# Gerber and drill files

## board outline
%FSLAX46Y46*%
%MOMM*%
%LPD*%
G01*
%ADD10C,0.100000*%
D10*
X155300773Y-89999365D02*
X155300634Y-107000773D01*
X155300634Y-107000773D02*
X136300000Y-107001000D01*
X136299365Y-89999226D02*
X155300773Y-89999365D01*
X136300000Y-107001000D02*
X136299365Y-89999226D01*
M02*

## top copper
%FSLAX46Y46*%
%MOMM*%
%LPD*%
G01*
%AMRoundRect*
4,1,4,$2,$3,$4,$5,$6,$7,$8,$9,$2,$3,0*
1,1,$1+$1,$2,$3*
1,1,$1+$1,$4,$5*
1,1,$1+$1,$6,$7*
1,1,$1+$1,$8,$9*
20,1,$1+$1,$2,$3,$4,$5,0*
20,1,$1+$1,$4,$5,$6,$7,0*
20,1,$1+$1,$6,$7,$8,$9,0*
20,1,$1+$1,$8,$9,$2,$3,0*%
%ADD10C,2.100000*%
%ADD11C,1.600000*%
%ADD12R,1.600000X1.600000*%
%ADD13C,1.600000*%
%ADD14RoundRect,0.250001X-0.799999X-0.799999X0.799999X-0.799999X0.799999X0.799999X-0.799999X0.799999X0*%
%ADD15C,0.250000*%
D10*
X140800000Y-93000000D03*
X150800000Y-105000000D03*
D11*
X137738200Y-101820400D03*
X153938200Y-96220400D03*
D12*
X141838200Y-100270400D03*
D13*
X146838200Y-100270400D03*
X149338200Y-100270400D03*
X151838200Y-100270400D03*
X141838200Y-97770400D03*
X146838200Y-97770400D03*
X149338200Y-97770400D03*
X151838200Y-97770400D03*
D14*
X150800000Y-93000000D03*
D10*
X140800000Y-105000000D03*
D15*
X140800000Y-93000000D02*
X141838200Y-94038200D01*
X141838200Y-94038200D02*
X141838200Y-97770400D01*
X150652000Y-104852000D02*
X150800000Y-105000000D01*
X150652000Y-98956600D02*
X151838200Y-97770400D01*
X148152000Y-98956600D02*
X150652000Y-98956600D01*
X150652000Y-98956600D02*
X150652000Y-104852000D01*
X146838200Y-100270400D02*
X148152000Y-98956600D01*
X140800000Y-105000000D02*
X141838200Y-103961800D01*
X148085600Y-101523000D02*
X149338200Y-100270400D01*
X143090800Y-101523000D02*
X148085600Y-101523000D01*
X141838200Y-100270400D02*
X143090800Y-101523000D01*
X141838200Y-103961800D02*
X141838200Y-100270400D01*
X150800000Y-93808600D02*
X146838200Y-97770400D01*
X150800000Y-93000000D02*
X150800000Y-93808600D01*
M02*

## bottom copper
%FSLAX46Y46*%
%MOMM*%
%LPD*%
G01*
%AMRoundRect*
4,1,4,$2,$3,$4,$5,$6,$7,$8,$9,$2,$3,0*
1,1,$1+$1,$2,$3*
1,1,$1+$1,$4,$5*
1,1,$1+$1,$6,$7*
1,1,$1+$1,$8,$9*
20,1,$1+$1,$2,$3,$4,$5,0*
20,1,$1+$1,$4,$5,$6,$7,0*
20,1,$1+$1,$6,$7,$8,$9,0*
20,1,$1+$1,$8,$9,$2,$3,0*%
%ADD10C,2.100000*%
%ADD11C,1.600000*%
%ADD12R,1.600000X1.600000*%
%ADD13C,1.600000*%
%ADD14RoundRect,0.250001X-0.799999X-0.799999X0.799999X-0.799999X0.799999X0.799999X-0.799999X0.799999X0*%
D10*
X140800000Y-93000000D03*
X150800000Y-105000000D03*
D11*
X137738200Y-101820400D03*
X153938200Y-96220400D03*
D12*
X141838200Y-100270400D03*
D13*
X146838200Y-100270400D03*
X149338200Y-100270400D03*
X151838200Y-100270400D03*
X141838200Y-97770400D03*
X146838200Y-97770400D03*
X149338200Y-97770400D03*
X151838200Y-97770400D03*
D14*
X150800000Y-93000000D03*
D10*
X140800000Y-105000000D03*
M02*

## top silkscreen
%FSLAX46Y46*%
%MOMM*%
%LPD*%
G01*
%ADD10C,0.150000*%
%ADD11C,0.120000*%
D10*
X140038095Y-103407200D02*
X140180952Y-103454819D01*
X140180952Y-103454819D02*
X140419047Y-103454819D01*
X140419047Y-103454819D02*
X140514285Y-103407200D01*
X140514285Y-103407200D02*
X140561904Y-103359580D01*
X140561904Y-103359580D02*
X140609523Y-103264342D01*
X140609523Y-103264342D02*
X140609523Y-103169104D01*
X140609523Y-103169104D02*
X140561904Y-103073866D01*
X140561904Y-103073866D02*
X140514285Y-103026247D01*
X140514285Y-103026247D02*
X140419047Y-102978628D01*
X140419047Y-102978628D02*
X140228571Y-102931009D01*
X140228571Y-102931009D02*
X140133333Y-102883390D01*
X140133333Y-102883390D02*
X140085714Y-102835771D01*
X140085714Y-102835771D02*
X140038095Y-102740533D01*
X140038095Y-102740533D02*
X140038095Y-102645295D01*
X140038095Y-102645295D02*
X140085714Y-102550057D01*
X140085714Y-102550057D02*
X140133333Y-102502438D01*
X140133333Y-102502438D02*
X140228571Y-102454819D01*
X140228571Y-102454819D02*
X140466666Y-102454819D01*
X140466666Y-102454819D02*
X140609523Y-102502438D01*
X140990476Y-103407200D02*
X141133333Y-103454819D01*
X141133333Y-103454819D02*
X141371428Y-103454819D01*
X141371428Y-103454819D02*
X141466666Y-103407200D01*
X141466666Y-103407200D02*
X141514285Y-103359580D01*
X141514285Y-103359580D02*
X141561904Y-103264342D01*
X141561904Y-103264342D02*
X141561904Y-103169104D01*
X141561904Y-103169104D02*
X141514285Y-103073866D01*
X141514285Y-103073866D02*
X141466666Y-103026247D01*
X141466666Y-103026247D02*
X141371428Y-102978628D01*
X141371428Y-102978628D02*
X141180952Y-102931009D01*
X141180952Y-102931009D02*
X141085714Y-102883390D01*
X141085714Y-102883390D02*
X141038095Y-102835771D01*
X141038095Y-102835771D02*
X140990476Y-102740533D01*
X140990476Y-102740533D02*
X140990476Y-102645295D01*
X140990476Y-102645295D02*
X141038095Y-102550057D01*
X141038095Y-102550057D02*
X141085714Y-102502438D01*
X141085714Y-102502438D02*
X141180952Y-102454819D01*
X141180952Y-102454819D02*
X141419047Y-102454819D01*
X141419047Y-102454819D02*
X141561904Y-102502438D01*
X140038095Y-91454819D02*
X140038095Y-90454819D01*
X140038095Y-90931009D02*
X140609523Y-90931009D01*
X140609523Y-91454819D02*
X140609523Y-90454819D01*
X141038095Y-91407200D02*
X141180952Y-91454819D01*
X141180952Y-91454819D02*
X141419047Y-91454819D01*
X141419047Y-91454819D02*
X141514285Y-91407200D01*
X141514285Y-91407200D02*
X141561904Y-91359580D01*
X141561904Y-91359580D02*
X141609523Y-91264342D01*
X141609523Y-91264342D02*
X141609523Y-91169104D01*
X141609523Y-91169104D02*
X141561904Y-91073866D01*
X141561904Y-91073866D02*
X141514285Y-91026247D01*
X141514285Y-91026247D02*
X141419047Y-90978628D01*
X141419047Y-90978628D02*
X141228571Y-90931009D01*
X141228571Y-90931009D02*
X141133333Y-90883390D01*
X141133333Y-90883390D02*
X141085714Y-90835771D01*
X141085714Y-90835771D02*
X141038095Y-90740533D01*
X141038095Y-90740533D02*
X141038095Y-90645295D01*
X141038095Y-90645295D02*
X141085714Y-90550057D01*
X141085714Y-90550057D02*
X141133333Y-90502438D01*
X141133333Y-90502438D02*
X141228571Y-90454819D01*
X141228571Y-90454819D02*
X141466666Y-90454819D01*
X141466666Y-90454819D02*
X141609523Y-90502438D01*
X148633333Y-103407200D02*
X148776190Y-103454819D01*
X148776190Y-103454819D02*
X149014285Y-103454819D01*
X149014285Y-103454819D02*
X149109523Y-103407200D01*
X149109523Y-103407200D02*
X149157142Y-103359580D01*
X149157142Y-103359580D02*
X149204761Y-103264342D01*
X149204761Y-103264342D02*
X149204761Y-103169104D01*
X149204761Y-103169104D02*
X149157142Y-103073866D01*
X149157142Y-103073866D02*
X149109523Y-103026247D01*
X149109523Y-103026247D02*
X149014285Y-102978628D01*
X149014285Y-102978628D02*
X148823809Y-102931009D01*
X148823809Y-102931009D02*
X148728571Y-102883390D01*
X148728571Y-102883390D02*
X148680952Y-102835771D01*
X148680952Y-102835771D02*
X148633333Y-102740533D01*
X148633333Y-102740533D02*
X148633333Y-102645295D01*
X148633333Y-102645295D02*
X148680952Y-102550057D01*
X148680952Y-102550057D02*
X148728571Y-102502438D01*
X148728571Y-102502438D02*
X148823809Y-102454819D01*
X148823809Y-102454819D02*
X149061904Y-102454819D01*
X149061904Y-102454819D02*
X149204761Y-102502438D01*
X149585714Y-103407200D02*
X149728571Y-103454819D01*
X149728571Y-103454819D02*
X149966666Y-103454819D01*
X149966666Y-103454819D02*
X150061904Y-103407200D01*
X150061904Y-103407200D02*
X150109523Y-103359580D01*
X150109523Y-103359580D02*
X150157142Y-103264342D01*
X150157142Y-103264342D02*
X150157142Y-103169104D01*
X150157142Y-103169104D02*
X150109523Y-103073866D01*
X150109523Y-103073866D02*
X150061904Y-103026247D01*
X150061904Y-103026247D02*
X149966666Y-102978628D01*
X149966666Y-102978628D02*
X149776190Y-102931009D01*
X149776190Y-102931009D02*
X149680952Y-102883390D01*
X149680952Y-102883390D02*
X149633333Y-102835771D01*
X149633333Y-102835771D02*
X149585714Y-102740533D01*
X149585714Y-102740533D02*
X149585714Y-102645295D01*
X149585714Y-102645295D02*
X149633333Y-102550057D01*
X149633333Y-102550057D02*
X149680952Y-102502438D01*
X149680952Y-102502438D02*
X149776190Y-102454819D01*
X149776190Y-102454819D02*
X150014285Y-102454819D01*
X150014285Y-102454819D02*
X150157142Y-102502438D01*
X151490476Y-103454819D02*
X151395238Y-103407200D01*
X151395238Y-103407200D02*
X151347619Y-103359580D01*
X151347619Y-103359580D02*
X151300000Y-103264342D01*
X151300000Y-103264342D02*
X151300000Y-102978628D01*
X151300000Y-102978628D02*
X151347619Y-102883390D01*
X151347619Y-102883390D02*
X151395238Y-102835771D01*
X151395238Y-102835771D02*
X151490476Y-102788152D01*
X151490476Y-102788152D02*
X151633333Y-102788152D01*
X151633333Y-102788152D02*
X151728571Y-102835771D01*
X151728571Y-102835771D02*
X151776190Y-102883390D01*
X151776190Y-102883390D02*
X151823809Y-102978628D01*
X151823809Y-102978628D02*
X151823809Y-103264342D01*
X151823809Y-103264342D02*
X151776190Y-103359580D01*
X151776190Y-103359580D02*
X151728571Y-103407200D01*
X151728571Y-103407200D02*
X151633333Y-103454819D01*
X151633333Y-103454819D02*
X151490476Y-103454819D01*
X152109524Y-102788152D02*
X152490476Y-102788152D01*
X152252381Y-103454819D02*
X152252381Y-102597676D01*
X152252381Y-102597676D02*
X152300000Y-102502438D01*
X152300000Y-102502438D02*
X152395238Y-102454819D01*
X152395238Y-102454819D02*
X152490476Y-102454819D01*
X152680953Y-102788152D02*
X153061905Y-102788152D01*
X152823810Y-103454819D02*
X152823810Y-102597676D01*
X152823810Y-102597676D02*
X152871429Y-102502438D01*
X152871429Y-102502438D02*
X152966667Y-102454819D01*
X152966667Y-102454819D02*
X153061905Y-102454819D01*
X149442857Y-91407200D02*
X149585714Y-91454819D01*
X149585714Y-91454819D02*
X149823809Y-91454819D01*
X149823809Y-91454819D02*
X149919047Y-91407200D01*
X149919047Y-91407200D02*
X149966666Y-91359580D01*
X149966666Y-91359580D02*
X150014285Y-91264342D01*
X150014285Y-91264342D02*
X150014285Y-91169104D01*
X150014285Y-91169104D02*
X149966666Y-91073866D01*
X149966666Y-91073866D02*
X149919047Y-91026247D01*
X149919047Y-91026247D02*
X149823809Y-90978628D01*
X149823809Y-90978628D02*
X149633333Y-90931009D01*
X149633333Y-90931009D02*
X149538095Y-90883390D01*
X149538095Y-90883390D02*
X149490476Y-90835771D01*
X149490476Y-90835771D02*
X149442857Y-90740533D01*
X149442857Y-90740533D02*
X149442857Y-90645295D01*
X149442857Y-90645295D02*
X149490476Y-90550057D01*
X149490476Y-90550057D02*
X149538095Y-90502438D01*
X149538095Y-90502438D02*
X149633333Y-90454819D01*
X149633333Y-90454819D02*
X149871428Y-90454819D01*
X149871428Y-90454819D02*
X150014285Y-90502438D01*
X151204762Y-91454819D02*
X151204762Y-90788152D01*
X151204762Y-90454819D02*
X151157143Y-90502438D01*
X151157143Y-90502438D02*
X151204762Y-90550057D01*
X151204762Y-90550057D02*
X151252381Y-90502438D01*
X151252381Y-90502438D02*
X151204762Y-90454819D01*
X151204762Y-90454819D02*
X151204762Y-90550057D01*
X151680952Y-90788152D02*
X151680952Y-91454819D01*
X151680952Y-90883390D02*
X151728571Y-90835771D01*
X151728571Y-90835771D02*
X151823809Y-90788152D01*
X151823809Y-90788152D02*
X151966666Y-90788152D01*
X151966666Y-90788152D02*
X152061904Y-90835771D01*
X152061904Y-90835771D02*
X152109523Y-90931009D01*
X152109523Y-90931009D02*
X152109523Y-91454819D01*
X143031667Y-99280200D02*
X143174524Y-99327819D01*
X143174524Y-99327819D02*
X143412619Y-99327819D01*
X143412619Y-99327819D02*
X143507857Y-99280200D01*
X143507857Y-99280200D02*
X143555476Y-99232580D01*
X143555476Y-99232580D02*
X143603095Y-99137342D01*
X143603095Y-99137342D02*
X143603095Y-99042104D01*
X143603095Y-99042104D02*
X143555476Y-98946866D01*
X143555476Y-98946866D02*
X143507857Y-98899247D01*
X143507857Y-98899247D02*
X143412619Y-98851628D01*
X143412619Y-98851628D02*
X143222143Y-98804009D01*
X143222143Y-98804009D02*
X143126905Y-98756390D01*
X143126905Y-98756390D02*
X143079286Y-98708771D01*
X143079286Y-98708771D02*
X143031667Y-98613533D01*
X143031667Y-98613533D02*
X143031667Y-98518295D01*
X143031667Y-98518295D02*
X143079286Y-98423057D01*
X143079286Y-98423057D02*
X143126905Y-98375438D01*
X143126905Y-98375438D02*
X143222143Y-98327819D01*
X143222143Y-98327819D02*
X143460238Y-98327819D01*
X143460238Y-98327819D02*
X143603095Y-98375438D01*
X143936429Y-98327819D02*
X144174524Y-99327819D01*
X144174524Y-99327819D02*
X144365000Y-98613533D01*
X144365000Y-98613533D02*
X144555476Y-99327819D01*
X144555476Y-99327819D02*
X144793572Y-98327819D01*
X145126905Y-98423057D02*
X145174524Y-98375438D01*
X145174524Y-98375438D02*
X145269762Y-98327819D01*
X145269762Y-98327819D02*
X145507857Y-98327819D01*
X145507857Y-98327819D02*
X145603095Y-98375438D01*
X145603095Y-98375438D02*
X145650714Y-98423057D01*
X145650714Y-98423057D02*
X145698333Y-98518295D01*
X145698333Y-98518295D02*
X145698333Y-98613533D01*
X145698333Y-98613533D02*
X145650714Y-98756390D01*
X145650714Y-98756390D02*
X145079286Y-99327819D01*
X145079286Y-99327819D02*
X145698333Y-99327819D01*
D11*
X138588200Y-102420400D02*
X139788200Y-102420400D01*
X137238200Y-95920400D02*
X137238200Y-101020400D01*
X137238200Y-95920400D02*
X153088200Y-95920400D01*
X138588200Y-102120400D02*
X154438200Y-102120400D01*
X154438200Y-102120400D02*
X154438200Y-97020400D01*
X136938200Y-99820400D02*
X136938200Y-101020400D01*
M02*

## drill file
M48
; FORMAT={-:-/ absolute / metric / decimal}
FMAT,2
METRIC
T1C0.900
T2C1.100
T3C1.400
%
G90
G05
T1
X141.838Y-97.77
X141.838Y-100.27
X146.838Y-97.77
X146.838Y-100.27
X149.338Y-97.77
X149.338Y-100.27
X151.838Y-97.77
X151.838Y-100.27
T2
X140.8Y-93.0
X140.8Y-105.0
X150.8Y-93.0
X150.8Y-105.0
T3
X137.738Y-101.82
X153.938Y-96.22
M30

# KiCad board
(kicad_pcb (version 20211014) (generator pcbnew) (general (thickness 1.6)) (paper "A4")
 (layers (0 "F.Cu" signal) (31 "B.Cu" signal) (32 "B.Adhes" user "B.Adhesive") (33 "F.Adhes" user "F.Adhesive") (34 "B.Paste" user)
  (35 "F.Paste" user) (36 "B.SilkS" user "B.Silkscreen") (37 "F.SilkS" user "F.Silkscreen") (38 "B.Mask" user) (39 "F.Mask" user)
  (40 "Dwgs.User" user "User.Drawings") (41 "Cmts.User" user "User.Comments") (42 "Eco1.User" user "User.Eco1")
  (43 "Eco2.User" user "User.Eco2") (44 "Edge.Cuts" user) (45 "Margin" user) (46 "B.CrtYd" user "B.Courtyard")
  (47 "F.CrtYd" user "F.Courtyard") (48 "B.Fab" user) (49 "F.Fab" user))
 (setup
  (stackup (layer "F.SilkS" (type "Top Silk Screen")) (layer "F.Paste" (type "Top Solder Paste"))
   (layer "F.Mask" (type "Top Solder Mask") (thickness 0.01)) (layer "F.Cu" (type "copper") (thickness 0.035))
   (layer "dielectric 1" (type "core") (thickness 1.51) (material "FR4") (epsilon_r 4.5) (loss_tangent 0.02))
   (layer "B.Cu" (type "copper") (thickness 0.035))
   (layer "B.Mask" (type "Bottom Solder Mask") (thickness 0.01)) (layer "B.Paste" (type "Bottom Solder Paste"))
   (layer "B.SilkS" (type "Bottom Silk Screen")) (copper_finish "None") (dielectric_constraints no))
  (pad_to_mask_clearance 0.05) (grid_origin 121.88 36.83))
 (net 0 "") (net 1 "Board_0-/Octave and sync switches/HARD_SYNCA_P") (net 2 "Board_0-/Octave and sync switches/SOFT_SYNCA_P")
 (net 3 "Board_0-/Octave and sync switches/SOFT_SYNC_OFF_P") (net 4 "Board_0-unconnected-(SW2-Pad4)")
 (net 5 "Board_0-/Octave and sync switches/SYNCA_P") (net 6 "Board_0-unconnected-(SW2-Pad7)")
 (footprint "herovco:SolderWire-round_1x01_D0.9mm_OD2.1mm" (layer "F.Cu") (at 140.8 93)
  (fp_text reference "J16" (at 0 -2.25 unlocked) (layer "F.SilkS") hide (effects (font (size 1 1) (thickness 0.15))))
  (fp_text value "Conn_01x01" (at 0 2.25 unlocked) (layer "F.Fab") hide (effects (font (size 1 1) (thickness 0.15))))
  (pad "1" thru_hole circle (at 0 0) (size 2.1 2.1) (drill 1.1) (layers *.Cu *.Mask)
   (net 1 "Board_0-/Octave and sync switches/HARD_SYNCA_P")))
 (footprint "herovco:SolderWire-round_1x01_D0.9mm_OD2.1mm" (layer "F.Cu") (at 150.8 105)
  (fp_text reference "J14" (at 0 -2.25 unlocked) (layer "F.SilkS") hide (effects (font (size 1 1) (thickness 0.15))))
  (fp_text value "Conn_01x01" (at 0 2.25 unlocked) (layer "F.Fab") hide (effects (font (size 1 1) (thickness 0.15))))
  (pad "1" thru_hole circle (at 0 0) (size 2.1 2.1) (drill 1.1) (layers *.Cu *.Mask)
   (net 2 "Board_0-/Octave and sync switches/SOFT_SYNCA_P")))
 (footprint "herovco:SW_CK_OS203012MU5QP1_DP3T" (layer "F.Cu") (at 141.8382 100.2704)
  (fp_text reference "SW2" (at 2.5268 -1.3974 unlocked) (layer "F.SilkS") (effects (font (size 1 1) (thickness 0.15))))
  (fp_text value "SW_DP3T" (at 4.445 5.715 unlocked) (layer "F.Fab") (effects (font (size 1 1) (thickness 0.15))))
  (fp_line (start -3.25 2.15) (end -2.05 2.15) (layer "F.SilkS") (width 0.12))
  (fp_line (start -4.6 -4.35) (end -4.6 0.75) (layer "F.SilkS") (width 0.12))
  (fp_line (start -4.6 -4.35) (end 11.25 -4.35) (layer "F.SilkS") (width 0.12))
  (fp_line (start -3.25 1.85) (end 12.6 1.85) (layer "F.SilkS") (width 0.12))
  (fp_line (start 12.6 1.85) (end 12.6 -3.25) (layer "F.SilkS") (width 0.12))
  (fp_line (start -4.9 -0.45) (end -4.9 0.75) (layer "F.SilkS") (width 0.12))
  (pad "" np_thru_hole circle (at -4.1 1.55 180) (size 1.6 1.6) (drill 1.4) (layers F&B.Cu *.Mask))
  (pad "" np_thru_hole circle (at 12.1 -4.05 180) (size 1.6 1.6) (drill 1.4) (layers F&B.Cu *.Mask))
  (pad "1" thru_hole rect (at 0 0 180) (size 1.6 1.6) (drill 0.9) (layers *.Cu *.Mask)
   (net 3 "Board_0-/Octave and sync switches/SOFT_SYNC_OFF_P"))
  (pad "2" thru_hole circle (at 5 0 180) (size 1.6 1.6) (drill 0.9) (layers *.Cu *.Mask)
   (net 2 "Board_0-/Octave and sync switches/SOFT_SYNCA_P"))
  (pad "3" thru_hole circle (at 7.5 0 180) (size 1.6 1.6) (drill 0.9) (layers *.Cu *.Mask)
   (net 3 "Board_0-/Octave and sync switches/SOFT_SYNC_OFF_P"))
  (pad "4" thru_hole circle (at 10 0 180) (size 1.6 1.6) (drill 0.9) (layers *.Cu *.Mask) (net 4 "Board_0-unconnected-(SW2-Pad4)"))
  (pad "5" thru_hole circle (at 0 -2.5 180) (size 1.6 1.6) (drill 0.9) (layers *.Cu *.Mask)
   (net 1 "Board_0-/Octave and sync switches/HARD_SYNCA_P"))
  (pad "6" thru_hole circle (at 5 -2.5 180) (size 1.6 1.6) (drill 0.9) (layers *.Cu *.Mask)
   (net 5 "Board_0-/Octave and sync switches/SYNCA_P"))
  (pad "7" thru_hole circle (at 7.5 -2.5 180) (size 1.6 1.6) (drill 0.9) (layers *.Cu *.Mask) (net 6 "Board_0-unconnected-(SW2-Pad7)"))
  (pad "8" thru_hole circle (at 10 -2.5 180) (size 1.6 1.6) (drill 0.9) (layers *.Cu *.Mask)
   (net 2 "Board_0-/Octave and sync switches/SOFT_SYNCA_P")))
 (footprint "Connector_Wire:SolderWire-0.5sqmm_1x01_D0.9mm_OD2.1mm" (layer "F.Cu") (at 150.8 93)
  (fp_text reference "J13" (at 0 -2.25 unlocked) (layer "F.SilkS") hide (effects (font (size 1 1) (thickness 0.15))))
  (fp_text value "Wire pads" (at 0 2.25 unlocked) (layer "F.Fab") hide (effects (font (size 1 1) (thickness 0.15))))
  (pad "1" thru_hole roundrect locked (at 0 0) (size 2.1 2.1) (drill 1.1) (layers *.Cu *.Mask) (roundrect_rratio 0.119048)
   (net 5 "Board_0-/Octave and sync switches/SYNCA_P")))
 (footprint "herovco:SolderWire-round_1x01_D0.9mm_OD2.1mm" (layer "F.Cu") (at 140.8 105)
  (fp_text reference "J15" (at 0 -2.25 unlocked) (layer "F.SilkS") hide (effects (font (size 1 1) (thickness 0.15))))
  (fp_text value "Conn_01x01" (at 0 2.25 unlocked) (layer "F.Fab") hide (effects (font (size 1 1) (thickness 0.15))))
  (pad "1" thru_hole circle (at 0 0) (size 2.1 2.1) (drill 1.1) (layers *.Cu *.Mask)
   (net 3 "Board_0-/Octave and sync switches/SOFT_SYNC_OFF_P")))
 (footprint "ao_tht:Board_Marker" (layer "F.Cu") (at 147.8 90)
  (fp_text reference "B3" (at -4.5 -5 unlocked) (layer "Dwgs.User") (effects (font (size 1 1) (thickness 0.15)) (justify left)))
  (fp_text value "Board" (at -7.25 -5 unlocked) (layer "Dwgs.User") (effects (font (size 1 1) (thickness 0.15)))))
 (gr_line (start 155.300773 89.999365) (end 155.300634 107.000773) (layer "Edge.Cuts") (width 0.1))
 (gr_line (start 155.300634 107.000773) (end 136.3 107.001) (layer "Edge.Cuts") (width 0.1))
 (gr_line (start 136.299365 89.999226) (end 155.300773 89.999365) (layer "Edge.Cuts") (width 0.1))
 (gr_line (start 136.3 107.001) (end 136.299365 89.999226) (layer "Edge.Cuts") (width 0.1))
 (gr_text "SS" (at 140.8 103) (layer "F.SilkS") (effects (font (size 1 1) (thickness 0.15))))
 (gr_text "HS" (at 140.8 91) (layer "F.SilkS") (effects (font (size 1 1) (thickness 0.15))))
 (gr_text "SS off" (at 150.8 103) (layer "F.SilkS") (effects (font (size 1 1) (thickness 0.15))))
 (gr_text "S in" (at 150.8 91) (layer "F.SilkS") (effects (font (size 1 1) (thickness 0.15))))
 (segment (start 140.8 93) (end 141.8382 94.0382) (width 0.25) (layer "F.Cu") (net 1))
 (segment (start 141.8382 94.0382) (end 141.8382 97.7704) (width 0.25) (layer "F.Cu") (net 1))
 (segment (start 150.652 104.852) (end 150.8 105) (width 0.25) (layer "F.Cu") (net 2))
 (segment (start 150.652 98.9566) (end 151.8382 97.7704) (width 0.25) (layer "F.Cu") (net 2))
 (segment (start 148.152 98.9566) (end 150.652 98.9566) (width 0.25) (layer "F.Cu") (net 2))
 (segment (start 150.652 98.9566) (end 150.652 104.852) (width 0.25) (layer "F.Cu") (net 2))
 (segment (start 146.8382 100.2704) (end 148.152 98.9566) (width 0.25) (layer "F.Cu") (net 2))
 (segment (start 140.8 105) (end 141.8382 103.9618) (width 0.25) (layer "F.Cu") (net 3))
 (segment (start 148.0856 101.523) (end 149.3382 100.2704) (width 0.25) (layer "F.Cu") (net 3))
 (segment (start 143.0908 101.523) (end 148.0856 101.523) (width 0.25) (layer "F.Cu") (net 3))
 (segment (start 141.8382 100.2704) (end 143.0908 101.523) (width 0.25) (layer "F.Cu") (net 3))
 (segment (start 141.8382 103.9618) (end 141.8382 100.2704) (width 0.25) (layer "F.Cu") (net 3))
 (segment (start 150.8 93.8086) (end 146.8382 97.7704) (width 0.25) (layer "F.Cu") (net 5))
 (segment (start 150.8 93) (end 150.8 93.8086) (width 0.25) (layer "F.Cu") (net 5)))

